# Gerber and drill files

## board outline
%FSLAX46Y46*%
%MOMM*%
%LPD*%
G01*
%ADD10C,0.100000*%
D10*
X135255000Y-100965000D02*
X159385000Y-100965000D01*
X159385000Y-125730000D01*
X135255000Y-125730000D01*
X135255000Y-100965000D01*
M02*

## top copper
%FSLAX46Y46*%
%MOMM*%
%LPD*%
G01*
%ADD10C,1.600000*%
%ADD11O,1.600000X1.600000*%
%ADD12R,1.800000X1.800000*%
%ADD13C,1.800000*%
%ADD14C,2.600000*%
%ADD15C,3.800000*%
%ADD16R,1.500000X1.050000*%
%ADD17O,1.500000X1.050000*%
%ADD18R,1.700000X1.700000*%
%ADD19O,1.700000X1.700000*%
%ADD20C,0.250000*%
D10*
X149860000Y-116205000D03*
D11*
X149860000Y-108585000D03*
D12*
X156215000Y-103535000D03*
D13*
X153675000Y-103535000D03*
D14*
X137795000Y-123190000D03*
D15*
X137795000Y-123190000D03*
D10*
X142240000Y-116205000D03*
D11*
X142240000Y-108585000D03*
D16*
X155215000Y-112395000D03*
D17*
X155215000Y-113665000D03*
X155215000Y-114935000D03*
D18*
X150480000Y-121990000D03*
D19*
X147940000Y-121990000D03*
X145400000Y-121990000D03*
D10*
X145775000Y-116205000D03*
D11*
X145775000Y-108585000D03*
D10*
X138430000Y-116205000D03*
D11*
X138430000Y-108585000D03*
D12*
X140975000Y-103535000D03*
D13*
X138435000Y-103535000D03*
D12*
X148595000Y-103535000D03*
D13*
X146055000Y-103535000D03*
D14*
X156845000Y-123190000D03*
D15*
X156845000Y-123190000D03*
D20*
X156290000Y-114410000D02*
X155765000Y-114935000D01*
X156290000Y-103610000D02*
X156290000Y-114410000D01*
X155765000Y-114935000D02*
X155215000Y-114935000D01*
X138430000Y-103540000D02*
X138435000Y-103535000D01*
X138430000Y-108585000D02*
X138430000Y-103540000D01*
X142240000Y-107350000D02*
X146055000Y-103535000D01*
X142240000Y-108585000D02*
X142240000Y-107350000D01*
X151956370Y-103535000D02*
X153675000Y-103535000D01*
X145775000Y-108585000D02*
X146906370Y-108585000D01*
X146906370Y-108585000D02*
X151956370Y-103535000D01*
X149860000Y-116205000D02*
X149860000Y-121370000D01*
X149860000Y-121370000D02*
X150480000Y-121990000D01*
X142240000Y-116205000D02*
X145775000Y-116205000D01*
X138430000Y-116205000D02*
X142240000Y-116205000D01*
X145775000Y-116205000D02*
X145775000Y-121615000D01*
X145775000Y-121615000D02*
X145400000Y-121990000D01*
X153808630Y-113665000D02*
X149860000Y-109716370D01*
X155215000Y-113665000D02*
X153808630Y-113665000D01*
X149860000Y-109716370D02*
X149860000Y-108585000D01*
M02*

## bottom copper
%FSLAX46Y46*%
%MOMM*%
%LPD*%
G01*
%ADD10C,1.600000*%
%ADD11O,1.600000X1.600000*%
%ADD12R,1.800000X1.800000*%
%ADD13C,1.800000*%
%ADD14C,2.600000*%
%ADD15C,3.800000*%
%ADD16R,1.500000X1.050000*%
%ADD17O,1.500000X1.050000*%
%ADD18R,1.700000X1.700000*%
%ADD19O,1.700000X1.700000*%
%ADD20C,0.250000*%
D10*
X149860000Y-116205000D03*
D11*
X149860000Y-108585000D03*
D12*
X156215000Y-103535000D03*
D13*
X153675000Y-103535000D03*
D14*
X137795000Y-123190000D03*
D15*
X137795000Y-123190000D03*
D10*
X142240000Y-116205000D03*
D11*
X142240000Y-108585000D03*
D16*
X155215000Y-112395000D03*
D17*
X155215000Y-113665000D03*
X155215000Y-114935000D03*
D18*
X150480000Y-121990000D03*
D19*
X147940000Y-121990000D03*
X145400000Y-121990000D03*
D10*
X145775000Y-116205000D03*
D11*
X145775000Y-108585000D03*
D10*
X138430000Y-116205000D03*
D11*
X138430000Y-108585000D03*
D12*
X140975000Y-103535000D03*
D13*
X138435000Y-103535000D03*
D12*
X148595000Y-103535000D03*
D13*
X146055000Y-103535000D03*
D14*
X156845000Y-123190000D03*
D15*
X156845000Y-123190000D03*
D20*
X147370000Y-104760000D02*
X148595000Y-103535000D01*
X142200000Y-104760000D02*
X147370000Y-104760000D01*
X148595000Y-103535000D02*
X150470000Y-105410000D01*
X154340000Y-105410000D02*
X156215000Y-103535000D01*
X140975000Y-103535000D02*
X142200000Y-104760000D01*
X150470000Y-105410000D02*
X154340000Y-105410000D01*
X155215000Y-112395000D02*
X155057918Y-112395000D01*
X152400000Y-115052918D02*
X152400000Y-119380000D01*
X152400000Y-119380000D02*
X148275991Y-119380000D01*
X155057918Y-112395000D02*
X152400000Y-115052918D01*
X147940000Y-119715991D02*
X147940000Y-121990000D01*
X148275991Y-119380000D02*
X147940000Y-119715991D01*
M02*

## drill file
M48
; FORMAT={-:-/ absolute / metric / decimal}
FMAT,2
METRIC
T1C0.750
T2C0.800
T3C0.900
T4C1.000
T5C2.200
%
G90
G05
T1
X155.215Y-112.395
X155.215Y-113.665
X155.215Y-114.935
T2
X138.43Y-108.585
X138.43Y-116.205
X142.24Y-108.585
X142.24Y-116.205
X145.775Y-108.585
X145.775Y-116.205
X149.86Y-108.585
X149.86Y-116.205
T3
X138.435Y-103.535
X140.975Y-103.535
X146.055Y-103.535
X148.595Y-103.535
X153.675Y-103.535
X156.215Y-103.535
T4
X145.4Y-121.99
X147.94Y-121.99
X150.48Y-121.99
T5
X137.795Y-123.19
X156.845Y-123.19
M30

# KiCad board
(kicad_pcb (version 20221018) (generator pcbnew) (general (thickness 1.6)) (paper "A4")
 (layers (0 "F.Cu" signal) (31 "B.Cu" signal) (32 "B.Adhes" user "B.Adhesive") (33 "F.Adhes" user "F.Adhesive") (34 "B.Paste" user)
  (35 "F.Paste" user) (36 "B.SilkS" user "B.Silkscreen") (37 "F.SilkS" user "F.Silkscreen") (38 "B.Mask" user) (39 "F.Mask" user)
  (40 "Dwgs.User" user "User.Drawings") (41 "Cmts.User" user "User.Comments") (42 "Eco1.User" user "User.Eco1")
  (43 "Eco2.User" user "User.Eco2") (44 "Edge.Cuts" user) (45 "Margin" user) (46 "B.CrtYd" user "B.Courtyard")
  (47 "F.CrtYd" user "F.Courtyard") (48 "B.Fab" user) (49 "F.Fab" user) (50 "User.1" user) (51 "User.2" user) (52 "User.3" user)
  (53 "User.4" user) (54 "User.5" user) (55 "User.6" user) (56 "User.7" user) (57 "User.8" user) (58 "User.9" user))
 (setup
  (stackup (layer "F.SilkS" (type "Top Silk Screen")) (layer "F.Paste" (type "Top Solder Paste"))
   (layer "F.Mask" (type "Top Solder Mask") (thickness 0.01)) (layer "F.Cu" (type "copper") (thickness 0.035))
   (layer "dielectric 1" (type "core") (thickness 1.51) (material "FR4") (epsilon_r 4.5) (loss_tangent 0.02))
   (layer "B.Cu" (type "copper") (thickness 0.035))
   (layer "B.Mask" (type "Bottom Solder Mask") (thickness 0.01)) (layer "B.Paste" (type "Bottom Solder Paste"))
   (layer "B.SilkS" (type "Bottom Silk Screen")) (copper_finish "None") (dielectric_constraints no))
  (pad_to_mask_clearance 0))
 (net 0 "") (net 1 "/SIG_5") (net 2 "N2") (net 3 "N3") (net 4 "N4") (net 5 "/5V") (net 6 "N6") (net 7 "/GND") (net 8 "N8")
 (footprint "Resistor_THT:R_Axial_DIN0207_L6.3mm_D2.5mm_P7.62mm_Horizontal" (layer "F.Cu") (at 149.86 116.205 90)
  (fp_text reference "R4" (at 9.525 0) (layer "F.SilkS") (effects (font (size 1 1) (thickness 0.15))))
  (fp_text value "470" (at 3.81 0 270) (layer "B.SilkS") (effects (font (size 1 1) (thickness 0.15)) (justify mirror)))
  (pad "1" thru_hole circle (at 0 0 90) (size 1.6 1.6) (drill 0.8) (layers "*.Cu" "*.Mask") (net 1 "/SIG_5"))
  (pad "2" thru_hole oval (at 7.62 0 90) (size 1.6 1.6) (drill 0.8) (layers "*.Cu" "*.Mask") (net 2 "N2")))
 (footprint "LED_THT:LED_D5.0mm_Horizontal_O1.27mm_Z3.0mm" (layer "F.Cu") (at 156.215 103.535 180)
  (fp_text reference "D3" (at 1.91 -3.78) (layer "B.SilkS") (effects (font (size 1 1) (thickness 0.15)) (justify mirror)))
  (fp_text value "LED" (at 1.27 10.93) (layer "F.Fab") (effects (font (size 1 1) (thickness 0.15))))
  (pad "1" thru_hole rect (at 0 0 180) (size 1.8 1.8) (drill 0.9) (layers "*.Cu" "*.Mask") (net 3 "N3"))
  (pad "2" thru_hole circle (at 2.54 0 180) (size 1.8 1.8) (drill 0.9) (layers "*.Cu" "*.Mask") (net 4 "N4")))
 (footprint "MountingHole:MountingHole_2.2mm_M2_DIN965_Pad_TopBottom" (layer "F.Cu") (at 137.795 123.19)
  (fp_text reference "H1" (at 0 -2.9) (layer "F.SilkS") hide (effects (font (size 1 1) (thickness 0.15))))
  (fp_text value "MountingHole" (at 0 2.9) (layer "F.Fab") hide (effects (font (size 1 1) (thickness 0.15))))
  (pad "1" thru_hole circle (at 0 0) (size 2.6 2.6) (drill 2.2) (layers "*.Cu" "*.Mask"))
  (pad "1" connect circle (at 0 0) (size 3.8 3.8) (layers "F.Cu" "F.Mask"))
  (pad "1" connect circle (at 0 0) (size 3.8 3.8) (layers "B.Cu" "B.Mask")))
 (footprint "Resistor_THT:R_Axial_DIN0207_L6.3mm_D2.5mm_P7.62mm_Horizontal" (layer "F.Cu") (at 142.24 116.205 90)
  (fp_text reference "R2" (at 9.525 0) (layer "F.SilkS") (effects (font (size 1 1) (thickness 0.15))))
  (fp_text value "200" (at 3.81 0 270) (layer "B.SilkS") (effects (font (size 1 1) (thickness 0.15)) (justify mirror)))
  (pad "1" thru_hole circle (at 0 0 90) (size 1.6 1.6) (drill 0.8) (layers "*.Cu" "*.Mask") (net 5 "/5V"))
  (pad "2" thru_hole oval (at 7.62 0 90) (size 1.6 1.6) (drill 0.8) (layers "*.Cu" "*.Mask") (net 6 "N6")))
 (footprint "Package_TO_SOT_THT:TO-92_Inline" (layer "F.Cu") (at 155.215 112.395 -90)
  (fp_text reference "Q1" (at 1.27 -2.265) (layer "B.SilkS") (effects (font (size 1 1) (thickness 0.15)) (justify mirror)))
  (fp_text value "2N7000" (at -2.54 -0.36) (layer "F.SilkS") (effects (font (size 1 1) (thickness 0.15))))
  (pad "1" thru_hole rect (at 0 0 270) (size 1.05 1.5) (drill 0.75) (layers "*.Cu" "*.Mask") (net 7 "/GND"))
  (pad "2" thru_hole oval (at 1.27 0 270) (size 1.05 1.5) (drill 0.75) (layers "*.Cu" "*.Mask") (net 2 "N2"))
  (pad "3" thru_hole oval (at 2.54 0 270) (size 1.05 1.5) (drill 0.75) (layers "*.Cu" "*.Mask") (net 3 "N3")))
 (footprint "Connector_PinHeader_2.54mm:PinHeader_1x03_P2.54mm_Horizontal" (layer "F.Cu") (at 150.48 121.99 -90)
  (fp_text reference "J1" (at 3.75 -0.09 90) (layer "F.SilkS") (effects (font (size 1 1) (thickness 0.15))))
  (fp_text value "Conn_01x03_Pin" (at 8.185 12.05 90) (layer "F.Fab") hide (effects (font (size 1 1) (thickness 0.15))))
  (pad "1" thru_hole rect (at 0 0 270) (size 1.7 1.7) (drill 1) (layers "*.Cu" "*.Mask") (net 1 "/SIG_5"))
  (pad "2" thru_hole oval (at 0 2.54 270) (size 1.7 1.7) (drill 1) (layers "*.Cu" "*.Mask") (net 7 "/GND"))
  (pad "3" thru_hole oval (at 0 5.08 270) (size 1.7 1.7) (drill 1) (layers "*.Cu" "*.Mask") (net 5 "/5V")))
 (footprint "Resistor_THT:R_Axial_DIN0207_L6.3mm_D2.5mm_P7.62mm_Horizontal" (layer "F.Cu") (at 145.775 116.205 90)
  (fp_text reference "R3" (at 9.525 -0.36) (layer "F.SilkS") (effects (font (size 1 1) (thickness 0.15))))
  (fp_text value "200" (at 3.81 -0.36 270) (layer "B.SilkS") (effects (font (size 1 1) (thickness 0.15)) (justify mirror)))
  (pad "1" thru_hole circle (at 0 0 90) (size 1.6 1.6) (drill 0.8) (layers "*.Cu" "*.Mask") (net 5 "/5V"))
  (pad "2" thru_hole oval (at 7.62 0 90) (size 1.6 1.6) (drill 0.8) (layers "*.Cu" "*.Mask") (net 4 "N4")))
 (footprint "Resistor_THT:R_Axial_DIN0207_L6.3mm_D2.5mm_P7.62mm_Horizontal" (layer "F.Cu") (at 138.43 116.205 90)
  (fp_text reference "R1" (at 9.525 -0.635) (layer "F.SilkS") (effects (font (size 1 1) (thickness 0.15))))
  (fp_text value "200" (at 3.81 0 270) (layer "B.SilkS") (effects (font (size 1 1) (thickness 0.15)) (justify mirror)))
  (pad "1" thru_hole circle (at 0 0 90) (size 1.6 1.6) (drill 0.8) (layers "*.Cu" "*.Mask") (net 5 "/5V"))
  (pad "2" thru_hole oval (at 7.62 0 90) (size 1.6 1.6) (drill 0.8) (layers "*.Cu" "*.Mask") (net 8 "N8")))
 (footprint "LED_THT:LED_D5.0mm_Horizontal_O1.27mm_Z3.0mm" (layer "F.Cu") (at 140.975 103.535 180)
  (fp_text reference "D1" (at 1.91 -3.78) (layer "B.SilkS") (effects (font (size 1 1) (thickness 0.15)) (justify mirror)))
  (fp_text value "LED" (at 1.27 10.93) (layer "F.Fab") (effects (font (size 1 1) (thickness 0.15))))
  (pad "1" thru_hole rect (at 0 0 180) (size 1.8 1.8) (drill 0.9) (layers "*.Cu" "*.Mask") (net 3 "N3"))
  (pad "2" thru_hole circle (at 2.54 0 180) (size 1.8 1.8) (drill 0.9) (layers "*.Cu" "*.Mask") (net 8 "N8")))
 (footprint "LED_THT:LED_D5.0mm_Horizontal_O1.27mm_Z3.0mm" (layer "F.Cu") (at 148.595 103.535 180)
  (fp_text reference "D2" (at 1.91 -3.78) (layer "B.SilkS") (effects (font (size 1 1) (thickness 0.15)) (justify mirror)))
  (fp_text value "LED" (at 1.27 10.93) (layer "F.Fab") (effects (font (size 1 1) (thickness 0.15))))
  (pad "1" thru_hole rect (at 0 0 180) (size 1.8 1.8) (drill 0.9) (layers "*.Cu" "*.Mask") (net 3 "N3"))
  (pad "2" thru_hole circle (at 2.54 0 180) (size 1.8 1.8) (drill 0.9) (layers "*.Cu" "*.Mask") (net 6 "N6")))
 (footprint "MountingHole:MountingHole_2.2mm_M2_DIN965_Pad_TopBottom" (layer "F.Cu") (at 156.845 123.19)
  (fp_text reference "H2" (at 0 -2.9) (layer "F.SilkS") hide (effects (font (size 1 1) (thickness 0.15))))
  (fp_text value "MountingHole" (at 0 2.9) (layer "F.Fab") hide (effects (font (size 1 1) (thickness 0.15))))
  (pad "1" thru_hole circle (at 0 0) (size 2.6 2.6) (drill 2.2) (layers "*.Cu" "*.Mask"))
  (pad "1" connect circle (at 0 0) (size 3.8 3.8) (layers "F.Cu" "F.Mask"))
  (pad "1" connect circle (at 0 0) (size 3.8 3.8) (layers "B.Cu" "B.Mask")))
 (gr_rect (start 135.255 100.965) (end 159.385 125.73) (stroke (width 0.1) (type default)) (fill none) (layer "Edge.Cuts"))
 (segment (start 156.29 114.41) (end 155.765 114.935) (width 0.25) (layer "F.Cu") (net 3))
 (segment (start 156.29 103.61) (end 156.29 114.41) (width 0.25) (layer "F.Cu") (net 3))
 (segment (start 155.765 114.935) (end 155.215 114.935) (width 0.25) (layer "F.Cu") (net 3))
 (segment (start 147.37 104.76) (end 148.595 103.535) (width 0.25) (layer "B.Cu") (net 3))
 (segment (start 142.2 104.76) (end 147.37 104.76) (width 0.25) (layer "B.Cu") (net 3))
 (segment (start 148.595 103.535) (end 150.47 105.41) (width 0.25) (layer "B.Cu") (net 3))
 (segment (start 154.34 105.41) (end 156.215 103.535) (width 0.25) (layer "B.Cu") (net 3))
 (segment (start 140.975 103.535) (end 142.2 104.76) (width 0.25) (layer "B.Cu") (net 3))
 (segment (start 150.47 105.41) (end 154.34 105.41) (width 0.25) (layer "B.Cu") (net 3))
 (segment (start 138.43 103.54) (end 138.435 103.535) (width 0.25) (layer "F.Cu") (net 8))
 (segment (start 138.43 108.585) (end 138.43 103.54) (width 0.25) (layer "F.Cu") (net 8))
 (segment (start 142.24 107.35) (end 146.055 103.535) (width 0.25) (layer "F.Cu") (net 6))
 (segment (start 142.24 108.585) (end 142.24 107.35) (width 0.25) (layer "F.Cu") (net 6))
 (segment (start 151.95637 103.535) (end 153.675 103.535) (width 0.25) (layer "F.Cu") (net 4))
 (segment (start 145.775 108.585) (end 146.90637 108.585) (width 0.25) (layer "F.Cu") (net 4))
 (segment (start 146.90637 108.585) (end 151.95637 103.535) (width 0.25) (layer "F.Cu") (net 4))
 (segment (start 149.86 116.205) (end 149.86 121.37) (width 0.25) (layer "F.Cu") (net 1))
 (segment (start 149.86 121.37) (end 150.48 121.99) (width 0.25) (layer "F.Cu") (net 1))
 (segment (start 155.215 112.395) (end 155.057918 112.395) (width 0.25) (layer "B.Cu") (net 7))
 (segment (start 152.4 115.052918) (end 152.4 119.38) (width 0.25) (layer "B.Cu") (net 7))
 (segment (start 152.4 119.38) (end 148.275991 119.38) (width 0.25) (layer "B.Cu") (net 7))
 (segment (start 155.057918 112.395) (end 152.4 115.052918) (width 0.25) (layer "B.Cu") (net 7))
 (segment (start 147.94 119.715991) (end 147.94 121.99) (width 0.25) (layer "B.Cu") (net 7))
 (segment (start 148.275991 119.38) (end 147.94 119.715991) (width 0.25) (layer "B.Cu") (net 7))
 (segment (start 142.24 116.205) (end 145.775 116.205) (width 0.25) (layer "F.Cu") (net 5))
 (segment (start 138.43 116.205) (end 142.24 116.205) (width 0.25) (layer "F.Cu") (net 5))
 (segment (start 145.775 116.205) (end 145.775 121.615) (width 0.25) (layer "F.Cu") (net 5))
 (segment (start 145.775 121.615) (end 145.4 121.99) (width 0.25) (layer "F.Cu") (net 5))
 (segment (start 153.80863 113.665) (end 149.86 109.71637) (width 0.25) (layer "F.Cu") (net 2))
 (segment (start 155.215 113.665) (end 153.80863 113.665) (width 0.25) (layer "F.Cu") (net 2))
 (segment (start 149.86 109.71637) (end 149.86 108.585) (width 0.25) (layer "F.Cu") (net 2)))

